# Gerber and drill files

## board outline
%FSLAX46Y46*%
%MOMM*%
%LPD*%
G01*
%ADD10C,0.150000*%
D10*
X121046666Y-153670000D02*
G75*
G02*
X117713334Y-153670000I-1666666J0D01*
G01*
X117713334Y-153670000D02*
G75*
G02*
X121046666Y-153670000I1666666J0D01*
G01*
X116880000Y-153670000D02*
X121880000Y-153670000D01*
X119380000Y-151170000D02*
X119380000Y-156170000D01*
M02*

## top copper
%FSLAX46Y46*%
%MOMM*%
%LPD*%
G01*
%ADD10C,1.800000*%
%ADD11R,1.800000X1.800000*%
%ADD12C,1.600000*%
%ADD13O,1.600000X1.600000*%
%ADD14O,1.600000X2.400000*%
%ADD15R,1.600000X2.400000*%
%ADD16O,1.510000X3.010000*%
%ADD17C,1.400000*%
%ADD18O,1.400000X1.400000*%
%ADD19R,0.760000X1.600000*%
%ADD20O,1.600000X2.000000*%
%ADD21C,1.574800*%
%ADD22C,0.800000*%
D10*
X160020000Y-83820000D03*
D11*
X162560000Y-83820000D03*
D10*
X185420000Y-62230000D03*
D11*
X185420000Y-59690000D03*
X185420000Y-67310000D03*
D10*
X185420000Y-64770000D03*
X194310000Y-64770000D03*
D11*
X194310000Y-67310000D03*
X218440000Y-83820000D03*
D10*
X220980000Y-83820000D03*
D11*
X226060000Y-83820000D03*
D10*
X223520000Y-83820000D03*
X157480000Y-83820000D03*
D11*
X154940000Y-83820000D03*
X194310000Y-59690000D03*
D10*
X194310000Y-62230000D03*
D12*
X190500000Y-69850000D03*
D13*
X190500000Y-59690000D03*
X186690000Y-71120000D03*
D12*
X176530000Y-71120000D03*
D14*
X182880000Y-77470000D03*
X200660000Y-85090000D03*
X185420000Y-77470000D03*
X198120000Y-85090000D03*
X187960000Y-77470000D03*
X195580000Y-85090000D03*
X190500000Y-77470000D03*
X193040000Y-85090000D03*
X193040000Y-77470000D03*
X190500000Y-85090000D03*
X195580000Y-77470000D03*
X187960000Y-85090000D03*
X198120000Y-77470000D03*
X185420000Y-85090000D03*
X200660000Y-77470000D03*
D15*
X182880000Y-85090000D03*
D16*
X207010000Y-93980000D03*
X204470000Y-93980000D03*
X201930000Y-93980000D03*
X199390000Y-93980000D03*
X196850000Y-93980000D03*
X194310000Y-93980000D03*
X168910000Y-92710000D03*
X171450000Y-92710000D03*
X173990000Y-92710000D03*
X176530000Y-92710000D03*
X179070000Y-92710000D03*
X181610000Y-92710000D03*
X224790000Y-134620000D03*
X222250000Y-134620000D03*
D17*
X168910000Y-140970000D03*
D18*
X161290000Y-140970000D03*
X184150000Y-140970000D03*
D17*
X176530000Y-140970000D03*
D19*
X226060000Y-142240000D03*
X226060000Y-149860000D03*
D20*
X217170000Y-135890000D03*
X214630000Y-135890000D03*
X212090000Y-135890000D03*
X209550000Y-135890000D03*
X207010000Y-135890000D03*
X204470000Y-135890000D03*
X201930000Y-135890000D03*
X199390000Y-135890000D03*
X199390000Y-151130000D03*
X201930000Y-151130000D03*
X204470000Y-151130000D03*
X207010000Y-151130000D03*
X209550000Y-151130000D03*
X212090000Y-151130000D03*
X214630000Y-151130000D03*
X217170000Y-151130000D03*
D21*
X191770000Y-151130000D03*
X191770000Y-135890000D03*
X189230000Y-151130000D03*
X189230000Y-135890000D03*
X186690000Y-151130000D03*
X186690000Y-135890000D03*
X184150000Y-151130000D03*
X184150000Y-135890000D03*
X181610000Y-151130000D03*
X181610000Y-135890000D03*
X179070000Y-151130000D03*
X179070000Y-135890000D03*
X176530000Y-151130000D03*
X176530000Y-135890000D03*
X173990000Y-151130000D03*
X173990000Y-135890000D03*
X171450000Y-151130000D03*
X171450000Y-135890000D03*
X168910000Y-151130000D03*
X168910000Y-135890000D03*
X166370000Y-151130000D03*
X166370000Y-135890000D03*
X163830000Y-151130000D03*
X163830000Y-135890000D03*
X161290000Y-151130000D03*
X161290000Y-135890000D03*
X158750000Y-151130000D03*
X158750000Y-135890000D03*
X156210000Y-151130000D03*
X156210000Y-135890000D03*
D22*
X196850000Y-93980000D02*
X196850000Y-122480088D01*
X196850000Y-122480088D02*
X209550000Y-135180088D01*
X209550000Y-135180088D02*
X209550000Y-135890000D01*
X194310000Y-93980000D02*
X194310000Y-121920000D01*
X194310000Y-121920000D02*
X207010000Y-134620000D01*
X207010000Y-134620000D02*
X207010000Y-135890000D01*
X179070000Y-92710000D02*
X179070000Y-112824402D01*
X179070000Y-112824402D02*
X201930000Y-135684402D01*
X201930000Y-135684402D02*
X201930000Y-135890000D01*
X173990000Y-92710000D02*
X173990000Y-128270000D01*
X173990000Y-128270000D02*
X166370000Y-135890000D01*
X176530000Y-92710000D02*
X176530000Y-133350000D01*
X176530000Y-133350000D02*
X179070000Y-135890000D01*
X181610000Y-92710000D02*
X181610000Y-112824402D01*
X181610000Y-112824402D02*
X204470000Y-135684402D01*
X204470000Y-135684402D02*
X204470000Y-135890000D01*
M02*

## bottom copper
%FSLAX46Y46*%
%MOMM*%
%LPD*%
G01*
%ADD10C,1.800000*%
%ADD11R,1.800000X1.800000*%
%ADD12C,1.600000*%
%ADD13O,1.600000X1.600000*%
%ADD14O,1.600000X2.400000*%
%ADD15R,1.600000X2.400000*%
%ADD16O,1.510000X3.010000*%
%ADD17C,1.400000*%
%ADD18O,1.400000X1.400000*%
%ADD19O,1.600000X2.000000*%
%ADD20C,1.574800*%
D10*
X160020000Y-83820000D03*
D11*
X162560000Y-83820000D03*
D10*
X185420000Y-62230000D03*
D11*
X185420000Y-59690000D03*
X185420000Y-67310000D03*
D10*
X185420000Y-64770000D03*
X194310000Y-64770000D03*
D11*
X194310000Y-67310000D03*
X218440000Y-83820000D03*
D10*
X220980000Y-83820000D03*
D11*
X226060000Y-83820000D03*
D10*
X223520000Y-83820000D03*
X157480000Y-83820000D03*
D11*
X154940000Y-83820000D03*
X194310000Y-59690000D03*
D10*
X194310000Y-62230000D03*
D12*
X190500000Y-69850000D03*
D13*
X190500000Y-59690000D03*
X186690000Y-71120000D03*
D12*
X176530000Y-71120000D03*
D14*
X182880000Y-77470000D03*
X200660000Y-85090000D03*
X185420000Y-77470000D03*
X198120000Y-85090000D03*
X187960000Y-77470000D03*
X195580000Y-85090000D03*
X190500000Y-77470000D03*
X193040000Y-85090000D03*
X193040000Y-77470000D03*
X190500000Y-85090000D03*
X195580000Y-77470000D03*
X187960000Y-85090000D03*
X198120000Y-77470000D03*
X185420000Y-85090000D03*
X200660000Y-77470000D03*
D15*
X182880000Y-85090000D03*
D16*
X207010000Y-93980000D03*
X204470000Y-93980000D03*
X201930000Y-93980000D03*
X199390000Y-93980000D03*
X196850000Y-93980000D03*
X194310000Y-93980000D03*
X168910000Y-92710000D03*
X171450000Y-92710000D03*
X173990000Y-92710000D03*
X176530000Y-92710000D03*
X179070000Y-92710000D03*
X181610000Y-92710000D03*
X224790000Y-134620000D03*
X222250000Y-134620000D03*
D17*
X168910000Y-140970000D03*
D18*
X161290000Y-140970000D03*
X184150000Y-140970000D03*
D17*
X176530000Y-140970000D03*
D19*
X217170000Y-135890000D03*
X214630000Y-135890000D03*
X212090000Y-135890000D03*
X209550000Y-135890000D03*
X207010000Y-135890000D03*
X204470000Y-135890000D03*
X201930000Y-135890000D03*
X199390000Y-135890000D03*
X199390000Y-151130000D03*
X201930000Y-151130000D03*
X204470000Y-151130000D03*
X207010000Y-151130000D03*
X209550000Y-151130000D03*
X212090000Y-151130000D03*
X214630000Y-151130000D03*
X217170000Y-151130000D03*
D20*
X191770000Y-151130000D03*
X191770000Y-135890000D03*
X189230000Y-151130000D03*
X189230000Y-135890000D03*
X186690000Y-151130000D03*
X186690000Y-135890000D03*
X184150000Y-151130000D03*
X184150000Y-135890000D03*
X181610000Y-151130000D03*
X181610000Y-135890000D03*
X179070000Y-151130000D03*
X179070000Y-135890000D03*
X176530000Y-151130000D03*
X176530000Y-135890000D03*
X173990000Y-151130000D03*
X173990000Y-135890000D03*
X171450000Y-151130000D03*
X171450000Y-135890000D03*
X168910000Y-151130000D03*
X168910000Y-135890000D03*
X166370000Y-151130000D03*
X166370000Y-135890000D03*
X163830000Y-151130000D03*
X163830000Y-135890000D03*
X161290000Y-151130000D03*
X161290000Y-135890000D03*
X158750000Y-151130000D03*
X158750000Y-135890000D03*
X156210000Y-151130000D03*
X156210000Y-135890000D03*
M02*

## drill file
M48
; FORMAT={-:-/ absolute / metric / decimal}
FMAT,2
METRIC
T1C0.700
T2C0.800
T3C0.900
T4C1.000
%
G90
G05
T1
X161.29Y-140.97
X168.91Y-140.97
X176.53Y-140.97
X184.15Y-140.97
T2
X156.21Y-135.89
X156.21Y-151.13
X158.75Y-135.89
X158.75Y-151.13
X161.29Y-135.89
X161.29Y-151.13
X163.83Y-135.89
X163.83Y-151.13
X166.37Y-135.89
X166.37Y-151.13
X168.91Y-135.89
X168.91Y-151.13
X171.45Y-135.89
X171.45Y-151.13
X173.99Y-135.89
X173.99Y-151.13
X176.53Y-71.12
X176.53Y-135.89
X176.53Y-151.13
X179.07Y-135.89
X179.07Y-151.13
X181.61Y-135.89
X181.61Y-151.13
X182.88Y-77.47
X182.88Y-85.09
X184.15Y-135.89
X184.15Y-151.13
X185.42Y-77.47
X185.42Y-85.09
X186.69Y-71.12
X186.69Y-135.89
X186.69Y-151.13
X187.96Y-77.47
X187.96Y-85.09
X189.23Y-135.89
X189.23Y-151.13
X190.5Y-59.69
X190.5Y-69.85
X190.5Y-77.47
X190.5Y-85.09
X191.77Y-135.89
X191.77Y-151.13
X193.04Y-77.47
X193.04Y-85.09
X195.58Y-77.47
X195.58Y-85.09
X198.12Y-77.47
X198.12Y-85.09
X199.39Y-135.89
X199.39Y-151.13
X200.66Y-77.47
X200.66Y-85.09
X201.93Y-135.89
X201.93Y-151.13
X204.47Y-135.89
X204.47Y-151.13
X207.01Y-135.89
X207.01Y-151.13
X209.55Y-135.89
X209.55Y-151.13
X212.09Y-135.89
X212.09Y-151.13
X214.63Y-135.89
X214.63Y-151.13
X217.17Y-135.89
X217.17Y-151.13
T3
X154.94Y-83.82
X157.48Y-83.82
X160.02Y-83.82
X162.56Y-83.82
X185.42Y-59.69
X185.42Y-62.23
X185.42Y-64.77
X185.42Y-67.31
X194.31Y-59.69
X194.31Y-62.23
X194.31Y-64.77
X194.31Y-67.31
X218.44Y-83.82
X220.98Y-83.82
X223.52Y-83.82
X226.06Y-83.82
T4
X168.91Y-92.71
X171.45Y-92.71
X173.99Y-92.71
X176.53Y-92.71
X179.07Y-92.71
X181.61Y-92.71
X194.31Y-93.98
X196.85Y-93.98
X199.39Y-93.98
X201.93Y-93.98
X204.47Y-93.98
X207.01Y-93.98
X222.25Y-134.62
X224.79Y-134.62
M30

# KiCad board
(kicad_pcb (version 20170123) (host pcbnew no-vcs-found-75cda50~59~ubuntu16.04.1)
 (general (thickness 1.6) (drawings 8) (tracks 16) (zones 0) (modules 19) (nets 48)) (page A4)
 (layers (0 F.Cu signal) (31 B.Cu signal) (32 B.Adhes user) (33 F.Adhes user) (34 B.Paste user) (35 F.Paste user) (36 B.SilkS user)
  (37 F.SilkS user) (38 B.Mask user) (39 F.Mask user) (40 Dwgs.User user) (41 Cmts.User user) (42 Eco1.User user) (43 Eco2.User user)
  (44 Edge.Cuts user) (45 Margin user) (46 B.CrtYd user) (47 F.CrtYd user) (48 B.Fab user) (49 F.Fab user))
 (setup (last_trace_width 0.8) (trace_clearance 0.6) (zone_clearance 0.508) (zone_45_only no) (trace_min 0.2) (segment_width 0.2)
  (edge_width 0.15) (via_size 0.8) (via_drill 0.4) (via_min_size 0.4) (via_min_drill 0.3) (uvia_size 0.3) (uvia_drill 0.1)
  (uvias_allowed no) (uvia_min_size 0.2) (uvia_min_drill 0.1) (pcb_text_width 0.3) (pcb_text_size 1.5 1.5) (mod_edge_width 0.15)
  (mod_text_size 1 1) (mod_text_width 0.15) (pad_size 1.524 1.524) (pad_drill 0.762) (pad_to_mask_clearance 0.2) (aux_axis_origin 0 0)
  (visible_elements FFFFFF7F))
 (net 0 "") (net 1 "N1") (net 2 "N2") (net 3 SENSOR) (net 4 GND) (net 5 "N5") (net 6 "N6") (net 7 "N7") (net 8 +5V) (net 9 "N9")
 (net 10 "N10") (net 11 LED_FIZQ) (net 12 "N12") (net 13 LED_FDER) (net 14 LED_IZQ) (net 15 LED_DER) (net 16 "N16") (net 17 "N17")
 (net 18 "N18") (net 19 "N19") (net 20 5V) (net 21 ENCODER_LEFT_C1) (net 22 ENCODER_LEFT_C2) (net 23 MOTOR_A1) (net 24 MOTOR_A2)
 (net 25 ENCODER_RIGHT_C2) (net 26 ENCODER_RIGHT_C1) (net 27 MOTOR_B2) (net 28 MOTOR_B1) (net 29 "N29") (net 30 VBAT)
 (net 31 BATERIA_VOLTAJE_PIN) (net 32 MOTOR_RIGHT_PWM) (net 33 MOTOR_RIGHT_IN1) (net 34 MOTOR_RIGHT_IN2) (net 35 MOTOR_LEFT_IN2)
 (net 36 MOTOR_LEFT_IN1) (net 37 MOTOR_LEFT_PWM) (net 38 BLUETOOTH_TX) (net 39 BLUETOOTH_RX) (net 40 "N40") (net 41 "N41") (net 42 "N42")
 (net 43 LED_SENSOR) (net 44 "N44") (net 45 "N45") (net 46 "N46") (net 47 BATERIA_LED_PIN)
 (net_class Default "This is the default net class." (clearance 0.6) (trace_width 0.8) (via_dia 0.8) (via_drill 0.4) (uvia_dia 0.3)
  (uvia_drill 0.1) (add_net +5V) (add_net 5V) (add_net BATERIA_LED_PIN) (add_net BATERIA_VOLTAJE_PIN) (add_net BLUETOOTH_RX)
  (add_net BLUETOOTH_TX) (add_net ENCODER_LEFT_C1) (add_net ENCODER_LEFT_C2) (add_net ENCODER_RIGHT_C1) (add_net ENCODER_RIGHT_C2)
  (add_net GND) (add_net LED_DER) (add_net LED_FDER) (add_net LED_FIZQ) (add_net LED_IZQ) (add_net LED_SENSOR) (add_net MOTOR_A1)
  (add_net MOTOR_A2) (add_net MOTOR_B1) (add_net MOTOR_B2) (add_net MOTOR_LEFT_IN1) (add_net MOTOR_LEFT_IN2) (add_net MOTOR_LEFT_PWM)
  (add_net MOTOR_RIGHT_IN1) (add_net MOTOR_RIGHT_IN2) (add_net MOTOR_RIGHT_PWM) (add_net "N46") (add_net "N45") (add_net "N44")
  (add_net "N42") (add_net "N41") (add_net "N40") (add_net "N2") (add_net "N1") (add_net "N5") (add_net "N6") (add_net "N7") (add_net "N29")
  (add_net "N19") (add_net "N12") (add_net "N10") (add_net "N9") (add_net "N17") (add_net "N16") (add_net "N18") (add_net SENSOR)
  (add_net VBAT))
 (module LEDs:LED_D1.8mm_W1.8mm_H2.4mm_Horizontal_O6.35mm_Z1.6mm (layer F.Cu) (at 162.56 83.82 180)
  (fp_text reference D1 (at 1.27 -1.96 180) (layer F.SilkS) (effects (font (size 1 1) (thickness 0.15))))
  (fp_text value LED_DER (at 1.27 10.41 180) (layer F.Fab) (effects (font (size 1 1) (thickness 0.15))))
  (pad 2 thru_hole circle (at 2.54 0 180) (size 1.8 1.8) (drill 0.9) (layers *.Cu *.Mask) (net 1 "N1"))
  (pad 1 thru_hole rect (at 0 0 180) (size 1.8 1.8) (drill 0.9) (layers *.Cu *.Mask) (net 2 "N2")))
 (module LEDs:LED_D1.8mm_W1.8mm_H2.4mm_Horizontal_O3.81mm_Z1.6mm (layer F.Cu) (at 185.42 59.69 270)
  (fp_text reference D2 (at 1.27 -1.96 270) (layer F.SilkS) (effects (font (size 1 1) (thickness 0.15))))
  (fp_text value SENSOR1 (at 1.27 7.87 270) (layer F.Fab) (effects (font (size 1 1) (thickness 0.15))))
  (pad 2 thru_hole circle (at 2.54 0 270) (size 1.8 1.8) (drill 0.9) (layers *.Cu *.Mask) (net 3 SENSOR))
  (pad 1 thru_hole rect (at 0 0 270) (size 1.8 1.8) (drill 0.9) (layers *.Cu *.Mask) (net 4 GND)))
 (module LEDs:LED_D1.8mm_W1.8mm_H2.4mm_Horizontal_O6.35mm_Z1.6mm (layer B.Cu) (at 185.42 67.31 90)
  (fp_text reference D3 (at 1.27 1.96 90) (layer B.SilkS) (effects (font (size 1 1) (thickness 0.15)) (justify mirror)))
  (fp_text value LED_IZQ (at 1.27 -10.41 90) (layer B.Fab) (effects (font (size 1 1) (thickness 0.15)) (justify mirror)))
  (pad 1 thru_hole rect (at 0 0 90) (size 1.8 1.8) (drill 0.9) (layers *.Cu *.Mask) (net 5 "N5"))
  (pad 2 thru_hole circle (at 2.54 0 90) (size 1.8 1.8) (drill 0.9) (layers *.Cu *.Mask) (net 1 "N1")))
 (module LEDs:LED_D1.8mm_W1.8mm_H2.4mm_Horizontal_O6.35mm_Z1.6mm (layer F.Cu) (at 194.31 67.31 90)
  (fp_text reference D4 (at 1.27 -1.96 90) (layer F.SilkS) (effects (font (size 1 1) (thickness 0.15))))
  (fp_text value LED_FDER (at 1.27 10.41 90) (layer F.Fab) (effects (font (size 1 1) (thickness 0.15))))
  (pad 2 thru_hole circle (at 2.54 0 90) (size 1.8 1.8) (drill 0.9) (layers *.Cu *.Mask) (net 1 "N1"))
  (pad 1 thru_hole rect (at 0 0 90) (size 1.8 1.8) (drill 0.9) (layers *.Cu *.Mask) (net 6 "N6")))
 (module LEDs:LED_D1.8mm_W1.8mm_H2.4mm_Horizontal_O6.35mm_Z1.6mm (layer B.Cu) (at 218.44 83.82)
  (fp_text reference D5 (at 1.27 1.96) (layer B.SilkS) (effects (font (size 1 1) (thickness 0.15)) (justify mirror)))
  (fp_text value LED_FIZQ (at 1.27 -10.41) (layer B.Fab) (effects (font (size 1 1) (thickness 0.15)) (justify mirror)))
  (pad 1 thru_hole rect (at 0 0) (size 1.8 1.8) (drill 0.9) (layers *.Cu *.Mask) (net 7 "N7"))
  (pad 2 thru_hole circle (at 2.54 0) (size 1.8 1.8) (drill 0.9) (layers *.Cu *.Mask) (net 1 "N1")))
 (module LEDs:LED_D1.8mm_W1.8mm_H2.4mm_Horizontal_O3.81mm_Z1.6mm (layer F.Cu) (at 226.06 83.82 180)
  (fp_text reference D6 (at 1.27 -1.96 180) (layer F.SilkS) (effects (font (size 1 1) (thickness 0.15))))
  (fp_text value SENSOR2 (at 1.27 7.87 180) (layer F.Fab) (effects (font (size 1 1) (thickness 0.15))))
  (pad 1 thru_hole rect (at 0 0 180) (size 1.8 1.8) (drill 0.9) (layers *.Cu *.Mask) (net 4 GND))
  (pad 2 thru_hole circle (at 2.54 0 180) (size 1.8 1.8) (drill 0.9) (layers *.Cu *.Mask) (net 3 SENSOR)))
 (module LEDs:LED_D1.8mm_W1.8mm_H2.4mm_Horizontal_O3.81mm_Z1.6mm (layer B.Cu) (at 154.94 83.82)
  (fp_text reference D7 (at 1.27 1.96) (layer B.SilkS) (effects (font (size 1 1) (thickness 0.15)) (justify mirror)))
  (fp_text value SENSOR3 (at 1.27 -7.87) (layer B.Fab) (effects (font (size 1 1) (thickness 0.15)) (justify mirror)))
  (pad 2 thru_hole circle (at 2.54 0) (size 1.8 1.8) (drill 0.9) (layers *.Cu *.Mask) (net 3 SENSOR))
  (pad 1 thru_hole rect (at 0 0) (size 1.8 1.8) (drill 0.9) (layers *.Cu *.Mask) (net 4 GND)))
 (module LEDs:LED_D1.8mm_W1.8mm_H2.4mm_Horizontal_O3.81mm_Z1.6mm (layer B.Cu) (at 194.31 59.69 270)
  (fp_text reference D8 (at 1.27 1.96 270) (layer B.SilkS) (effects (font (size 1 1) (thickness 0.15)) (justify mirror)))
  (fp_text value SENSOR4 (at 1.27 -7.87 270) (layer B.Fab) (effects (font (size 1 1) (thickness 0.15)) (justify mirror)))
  (pad 1 thru_hole rect (at 0 0 270) (size 1.8 1.8) (drill 0.9) (layers *.Cu *.Mask) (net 4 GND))
  (pad 2 thru_hole circle (at 2.54 0 270) (size 1.8 1.8) (drill 0.9) (layers *.Cu *.Mask) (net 3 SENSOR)))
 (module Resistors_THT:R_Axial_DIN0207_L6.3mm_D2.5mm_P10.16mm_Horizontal (layer F.Cu) (at 190.5 69.85 90)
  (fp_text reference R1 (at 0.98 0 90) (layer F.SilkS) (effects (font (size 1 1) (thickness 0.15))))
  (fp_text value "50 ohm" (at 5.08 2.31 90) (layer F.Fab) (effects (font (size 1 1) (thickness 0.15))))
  (pad 1 thru_hole circle (at 0 0 90) (size 1.6 1.6) (drill 0.8) (layers *.Cu *.Mask) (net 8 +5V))
  (pad 2 thru_hole oval (at 10.16 0 90) (size 1.6 1.6) (drill 0.8) (layers *.Cu *.Mask) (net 1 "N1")))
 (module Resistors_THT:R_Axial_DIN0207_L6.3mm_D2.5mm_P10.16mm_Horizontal (layer F.Cu) (at 176.53 71.12)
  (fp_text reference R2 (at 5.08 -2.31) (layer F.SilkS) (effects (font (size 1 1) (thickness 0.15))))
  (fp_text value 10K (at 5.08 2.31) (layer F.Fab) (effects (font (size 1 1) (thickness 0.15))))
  (pad 2 thru_hole oval (at 10.16 0) (size 1.6 1.6) (drill 0.8) (layers *.Cu *.Mask) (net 8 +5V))
  (pad 1 thru_hole circle (at 0 0) (size 1.6 1.6) (drill 0.8) (layers *.Cu *.Mask) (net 3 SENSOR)))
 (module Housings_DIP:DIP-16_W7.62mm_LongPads (layer F.Cu) (at 182.88 85.09 90)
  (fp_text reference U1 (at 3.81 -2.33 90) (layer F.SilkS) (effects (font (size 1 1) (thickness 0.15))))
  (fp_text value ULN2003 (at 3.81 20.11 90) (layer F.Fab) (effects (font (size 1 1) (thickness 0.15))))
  (pad 16 thru_hole oval (at 7.62 0 90) (size 2.4 1.6) (drill 0.8) (layers *.Cu *.Mask) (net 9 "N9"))
  (pad 8 thru_hole oval (at 0 17.78 90) (size 2.4 1.6) (drill 0.8) (layers *.Cu *.Mask) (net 4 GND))
  (pad 15 thru_hole oval (at 7.62 2.54 90) (size 2.4 1.6) (drill 0.8) (layers *.Cu *.Mask) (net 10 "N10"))
  (pad 7 thru_hole oval (at 0 15.24 90) (size 2.4 1.6) (drill 0.8) (layers *.Cu *.Mask) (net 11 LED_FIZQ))
  (pad 14 thru_hole oval (at 7.62 5.08 90) (size 2.4 1.6) (drill 0.8) (layers *.Cu *.Mask) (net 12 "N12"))
  (pad 6 thru_hole oval (at 0 12.7 90) (size 2.4 1.6) (drill 0.8) (layers *.Cu *.Mask) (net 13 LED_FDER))
  (pad 13 thru_hole oval (at 7.62 7.62 90) (size 2.4 1.6) (drill 0.8) (layers *.Cu *.Mask) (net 2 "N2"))
  (pad 5 thru_hole oval (at 0 10.16 90) (size 2.4 1.6) (drill 0.8) (layers *.Cu *.Mask) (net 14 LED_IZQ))
  (pad 12 thru_hole oval (at 7.62 10.16 90) (size 2.4 1.6) (drill 0.8) (layers *.Cu *.Mask) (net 5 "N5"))
  (pad 4 thru_hole oval (at 0 7.62 90) (size 2.4 1.6) (drill 0.8) (layers *.Cu *.Mask) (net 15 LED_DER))
  (pad 11 thru_hole oval (at 7.62 12.7 90) (size 2.4 1.6) (drill 0.8) (layers *.Cu *.Mask) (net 6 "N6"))
  (pad 3 thru_hole oval (at 0 5.08 90) (size 2.4 1.6) (drill 0.8) (layers *.Cu *.Mask) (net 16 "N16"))
  (pad 10 thru_hole oval (at 7.62 15.24 90) (size 2.4 1.6) (drill 0.8) (layers *.Cu *.Mask) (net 7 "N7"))
  (pad 2 thru_hole oval (at 0 2.54 90) (size 2.4 1.6) (drill 0.8) (layers *.Cu *.Mask) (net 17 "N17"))
  (pad 9 thru_hole oval (at 7.62 17.78 90) (size 2.4 1.6) (drill 0.8) (layers *.Cu *.Mask) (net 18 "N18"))
  (pad 1 thru_hole rect (at 0 0 90) (size 2.4 1.6) (drill 0.8) (layers *.Cu *.Mask) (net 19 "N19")))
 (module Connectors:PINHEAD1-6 (layer F.Cu) (at 194.31 93.98)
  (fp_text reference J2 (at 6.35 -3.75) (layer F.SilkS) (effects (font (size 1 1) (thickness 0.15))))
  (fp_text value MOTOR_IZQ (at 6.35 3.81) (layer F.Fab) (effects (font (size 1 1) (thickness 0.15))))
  (pad 6 thru_hole oval (at 12.7 0) (size 1.51 3.01) (drill 1) (layers *.Cu *.Mask) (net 4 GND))
  (pad 5 thru_hole oval (at 10.16 0) (size 1.51 3.01) (drill 1) (layers *.Cu *.Mask) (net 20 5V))
  (pad 4 thru_hole oval (at 7.62 0) (size 1.51 3.01) (drill 1) (layers *.Cu *.Mask) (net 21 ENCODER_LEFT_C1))
  (pad 3 thru_hole oval (at 5.08 0) (size 1.51 3.01) (drill 1) (layers *.Cu *.Mask) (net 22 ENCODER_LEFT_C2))
  (pad 2 thru_hole oval (at 2.54 0) (size 1.51 3.01) (drill 1) (layers *.Cu *.Mask) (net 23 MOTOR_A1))
  (pad 1 thru_hole oval (at 0 0) (size 1.51 3.01) (drill 1) (layers *.Cu *.Mask) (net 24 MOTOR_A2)))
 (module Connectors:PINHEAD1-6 (layer F.Cu) (at 168.91 92.71)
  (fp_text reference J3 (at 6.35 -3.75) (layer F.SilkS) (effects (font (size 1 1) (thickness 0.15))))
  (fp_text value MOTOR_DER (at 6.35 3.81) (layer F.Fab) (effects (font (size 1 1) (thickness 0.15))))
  (pad 1 thru_hole oval (at 0 0) (size 1.51 3.01) (drill 1) (layers *.Cu *.Mask) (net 4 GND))
  (pad 2 thru_hole oval (at 2.54 0) (size 1.51 3.01) (drill 1) (layers *.Cu *.Mask) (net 20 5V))
  (pad 3 thru_hole oval (at 5.08 0) (size 1.51 3.01) (drill 1) (layers *.Cu *.Mask) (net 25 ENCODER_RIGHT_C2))
  (pad 4 thru_hole oval (at 7.62 0) (size 1.51 3.01) (drill 1) (layers *.Cu *.Mask) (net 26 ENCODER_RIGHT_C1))
  (pad 5 thru_hole oval (at 10.16 0) (size 1.51 3.01) (drill 1) (layers *.Cu *.Mask) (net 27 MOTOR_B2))
  (pad 6 thru_hole oval (at 12.7 0) (size 1.51 3.01) (drill 1) (layers *.Cu *.Mask) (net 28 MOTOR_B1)))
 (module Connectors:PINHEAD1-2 (layer F.Cu) (at 222.25 134.62)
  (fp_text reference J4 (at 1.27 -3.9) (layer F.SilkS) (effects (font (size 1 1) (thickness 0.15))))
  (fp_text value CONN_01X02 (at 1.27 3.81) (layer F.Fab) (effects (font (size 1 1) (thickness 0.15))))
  (pad 2 thru_hole oval (at 2.54 0) (size 1.51 3.01) (drill 1) (layers *.Cu *.Mask) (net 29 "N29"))
  (pad 1 thru_hole oval (at 0 0) (size 1.51 3.01) (drill 1) (layers *.Cu *.Mask) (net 4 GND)))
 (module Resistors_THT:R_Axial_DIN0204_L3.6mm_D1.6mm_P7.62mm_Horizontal (layer F.Cu) (at 168.91 140.97 180)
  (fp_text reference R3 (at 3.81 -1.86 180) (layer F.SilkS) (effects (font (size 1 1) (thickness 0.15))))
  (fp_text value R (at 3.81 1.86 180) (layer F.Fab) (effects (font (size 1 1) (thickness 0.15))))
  (pad 1 thru_hole circle (at 0 0 180) (size 1.4 1.4) (drill 0.7) (layers *.Cu *.Mask) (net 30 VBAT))
  (pad 2 thru_hole oval (at 7.62 0 180) (size 1.4 1.4) (drill 0.7) (layers *.Cu *.Mask) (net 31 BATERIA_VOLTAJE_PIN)))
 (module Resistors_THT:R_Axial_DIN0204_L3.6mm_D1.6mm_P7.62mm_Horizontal (layer F.Cu) (at 176.53 140.97)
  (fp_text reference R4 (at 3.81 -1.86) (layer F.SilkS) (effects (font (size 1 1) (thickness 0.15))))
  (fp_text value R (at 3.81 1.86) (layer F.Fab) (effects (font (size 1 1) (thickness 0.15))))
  (pad 2 thru_hole oval (at 7.62 0) (size 1.4 1.4) (drill 0.7) (layers *.Cu *.Mask) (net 4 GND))
  (pad 1 thru_hole circle (at 0 0) (size 1.4 1.4) (drill 0.7) (layers *.Cu *.Mask) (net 31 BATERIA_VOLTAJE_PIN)))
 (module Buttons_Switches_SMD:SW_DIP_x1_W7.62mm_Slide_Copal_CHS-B (layer F.Cu) (at 226.06 146.05 90)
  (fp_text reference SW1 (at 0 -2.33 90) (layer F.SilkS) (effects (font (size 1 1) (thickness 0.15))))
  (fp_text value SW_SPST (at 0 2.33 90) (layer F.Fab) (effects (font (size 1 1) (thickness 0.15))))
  (pad 2 smd rect (at 3.81 0 90) (size 1.6 0.76) (layers F.Cu F.Paste F.Mask) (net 30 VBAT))
  (pad 1 smd rect (at -3.81 0 90) (size 1.6 0.76) (layers F.Cu F.Paste F.Mask) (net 29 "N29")))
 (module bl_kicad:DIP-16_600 (layer F.Cu) (at 217.17 135.89 270)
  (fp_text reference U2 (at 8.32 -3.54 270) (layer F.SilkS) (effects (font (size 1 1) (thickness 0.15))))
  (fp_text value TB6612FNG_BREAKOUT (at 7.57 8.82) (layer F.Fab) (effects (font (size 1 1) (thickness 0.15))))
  (pad 1 thru_hole oval (at 0 0 270) (size 2 1.6) (drill 0.8) (layers *.Cu *.Mask F.SilkS) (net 30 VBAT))
  (pad 2 thru_hole oval (at 0 2.54 270) (size 2 1.6) (drill 0.8) (layers *.Cu *.Mask F.SilkS) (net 20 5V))
  (pad 3 thru_hole oval (at 0 5.08 270) (size 2 1.6) (drill 0.8) (layers *.Cu *.Mask F.SilkS) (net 4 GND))
  (pad 4 thru_hole oval (at 0 7.62 270) (size 2 1.6) (drill 0.8) (layers *.Cu *.Mask F.SilkS) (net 23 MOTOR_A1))
  (pad 5 thru_hole oval (at 0 10.16 270) (size 2 1.6) (drill 0.8) (layers *.Cu *.Mask F.SilkS) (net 24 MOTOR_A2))
  (pad 6 thru_hole oval (at 0 12.7 270) (size 2 1.6) (drill 0.8) (layers *.Cu *.Mask F.SilkS) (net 28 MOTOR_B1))
  (pad 7 thru_hole oval (at 0 15.24 270) (size 2 1.6) (drill 0.8) (layers *.Cu *.Mask F.SilkS) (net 27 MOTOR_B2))
  (pad 8 thru_hole oval (at 0 17.78 270) (size 2 1.6) (drill 0.8) (layers *.Cu *.Mask F.SilkS) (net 4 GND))
  (pad 9 thru_hole oval (at 15.24 17.78 270) (size 2 1.6) (drill 0.8) (layers *.Cu *.Mask F.SilkS) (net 4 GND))
  (pad 10 thru_hole oval (at 15.24 15.24 270) (size 2 1.6) (drill 0.8) (layers *.Cu *.Mask F.SilkS) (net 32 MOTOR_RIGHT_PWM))
  (pad 11 thru_hole oval (at 15.24 12.7 270) (size 2 1.6) (drill 0.8) (layers *.Cu *.Mask F.SilkS) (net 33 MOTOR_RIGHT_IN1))
  (pad 12 thru_hole oval (at 15.24 10.16 270) (size 2 1.6) (drill 0.8) (layers *.Cu *.Mask F.SilkS) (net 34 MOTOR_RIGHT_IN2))
  (pad 13 thru_hole oval (at 15.24 7.62 270) (size 2 1.6) (drill 0.8) (layers *.Cu *.Mask F.SilkS) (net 20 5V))
  (pad 14 thru_hole oval (at 15.24 5.08 270) (size 2 1.6) (drill 0.8) (layers *.Cu *.Mask F.SilkS) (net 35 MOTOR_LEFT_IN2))
  (pad 15 thru_hole oval (at 15.24 2.54 270) (size 2 1.6) (drill 0.8) (layers *.Cu *.Mask F.SilkS) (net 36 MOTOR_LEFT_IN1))
  (pad 16 thru_hole oval (at 15.24 0 270) (size 2 1.6) (drill 0.8) (layers *.Cu *.Mask F.SilkS) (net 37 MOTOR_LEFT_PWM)))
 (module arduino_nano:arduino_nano (layer F.Cu) (at 173.99 143.51 180)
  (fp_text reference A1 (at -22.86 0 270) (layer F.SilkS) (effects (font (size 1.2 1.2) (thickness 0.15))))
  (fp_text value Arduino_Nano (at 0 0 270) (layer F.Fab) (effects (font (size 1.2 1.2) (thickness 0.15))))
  (pad 30 thru_hole circle (at -17.78 -7.62 180) (size 1.5748 1.5748) (drill 0.8) (layers *.Cu *.Mask F.SilkS) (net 30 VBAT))
  (pad 1 thru_hole circle (at -17.78 7.62 180) (size 1.5748 1.5748) (drill 0.8) (layers *.Cu *.Mask F.SilkS) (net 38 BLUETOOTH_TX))
  (pad 29 thru_hole circle (at -15.24 -7.62 180) (size 1.5748 1.5748) (drill 0.8) (layers *.Cu *.Mask F.SilkS) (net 4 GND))
  (pad 2 thru_hole circle (at -15.24 7.62 180) (size 1.5748 1.5748) (drill 0.8) (layers *.Cu *.Mask F.SilkS) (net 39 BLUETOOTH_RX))
  (pad 28 thru_hole circle (at -12.7 -7.62 180) (size 1.5748 1.5748) (drill 0.8) (layers *.Cu *.Mask F.SilkS))
  (pad 3 thru_hole circle (at -12.7 7.62 180) (size 1.5748 1.5748) (drill 0.8) (layers *.Cu *.Mask F.SilkS) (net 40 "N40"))
  (pad 27 thru_hole circle (at -10.16 -7.62 180) (size 1.5748 1.5748) (drill 0.8) (layers *.Cu *.Mask F.SilkS) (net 20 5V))
  (pad 4 thru_hole circle (at -10.16 7.62 180) (size 1.5748 1.5748) (drill 0.8) (layers *.Cu *.Mask F.SilkS) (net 4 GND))
  (pad 26 thru_hole circle (at -7.62 -7.62 180) (size 1.5748 1.5748) (drill 0.8) (layers *.Cu *.Mask F.SilkS) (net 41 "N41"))
  (pad 5 thru_hole circle (at -7.62 7.62 180) (size 1.5748 1.5748) (drill 0.8) (layers *.Cu *.Mask F.SilkS) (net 21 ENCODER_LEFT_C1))
  (pad 25 thru_hole circle (at -5.08 -7.62 180) (size 1.5748 1.5748) (drill 0.8) (layers *.Cu *.Mask F.SilkS) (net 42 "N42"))
  (pad 6 thru_hole circle (at -5.08 7.62 180) (size 1.5748 1.5748) (drill 0.8) (layers *.Cu *.Mask F.SilkS) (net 26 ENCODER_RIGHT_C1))
  (pad 24 thru_hole circle (at -2.54 -7.62 180) (size 1.5748 1.5748) (drill 0.8) (layers *.Cu *.Mask F.SilkS) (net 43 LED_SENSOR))
  (pad 7 thru_hole circle (at -2.54 7.62 180) (size 1.5748 1.5748) (drill 0.8) (layers *.Cu *.Mask F.SilkS) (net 35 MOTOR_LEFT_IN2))
  (pad 23 thru_hole circle (at 0 -7.62 180) (size 1.5748 1.5748) (drill 0.8) (layers *.Cu *.Mask F.SilkS) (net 13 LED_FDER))
  (pad 8 thru_hole circle (at 0 7.62 180) (size 1.5748 1.5748) (drill 0.8) (layers *.Cu *.Mask F.SilkS) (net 37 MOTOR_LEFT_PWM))
  (pad 22 thru_hole circle (at 2.54 -7.62 180) (size 1.5748 1.5748) (drill 0.8) (layers *.Cu *.Mask F.SilkS) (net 11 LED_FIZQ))
  (pad 9 thru_hole circle (at 2.54 7.62 180) (size 1.5748 1.5748) (drill 0.8) (layers *.Cu *.Mask F.SilkS) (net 32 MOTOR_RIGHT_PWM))
  (pad 21 thru_hole circle (at 5.08 -7.62 180) (size 1.5748 1.5748) (drill 0.8) (layers *.Cu *.Mask F.SilkS) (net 15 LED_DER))
  (pad 10 thru_hole circle (at 5.08 7.62 180) (size 1.5748 1.5748) (drill 0.8) (layers *.Cu *.Mask F.SilkS) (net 33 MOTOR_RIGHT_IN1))
  (pad 20 thru_hole circle (at 7.62 -7.62 180) (size 1.5748 1.5748) (drill 0.8) (layers *.Cu *.Mask F.SilkS) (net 14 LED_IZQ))
  (pad 11 thru_hole circle (at 7.62 7.62 180) (size 1.5748 1.5748) (drill 0.8) (layers *.Cu *.Mask F.SilkS) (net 25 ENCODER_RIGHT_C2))
  (pad 19 thru_hole circle (at 10.16 -7.62 180) (size 1.5748 1.5748) (drill 0.8) (layers *.Cu *.Mask F.SilkS) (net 31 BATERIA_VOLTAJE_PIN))
  (pad 12 thru_hole circle (at 10.16 7.62 180) (size 1.5748 1.5748) (drill 0.8) (layers *.Cu *.Mask F.SilkS) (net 36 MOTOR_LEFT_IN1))
  (pad 18 thru_hole circle (at 12.7 -7.62 180) (size 1.5748 1.5748) (drill 0.8) (layers *.Cu *.Mask F.SilkS) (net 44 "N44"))
  (pad 13 thru_hole circle (at 12.7 7.62 180) (size 1.5748 1.5748) (drill 0.8) (layers *.Cu *.Mask F.SilkS) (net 34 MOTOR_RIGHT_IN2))
  (pad 17 thru_hole circle (at 15.24 -7.62 180) (size 1.5748 1.5748) (drill 0.8) (layers *.Cu *.Mask F.SilkS) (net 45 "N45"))
  (pad 14 thru_hole circle (at 15.24 7.62 180) (size 1.5748 1.5748) (drill 0.8) (layers *.Cu *.Mask F.SilkS) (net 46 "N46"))
  (pad 16 thru_hole circle (at 17.78 -7.62 180) (size 1.5748 1.5748) (drill 0.8) (layers *.Cu *.Mask F.SilkS) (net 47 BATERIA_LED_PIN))
  (pad 15 thru_hole circle (at 17.78 7.62 180) (size 1.5748 1.5748) (drill 0.8) (layers *.Cu *.Mask F.SilkS) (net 22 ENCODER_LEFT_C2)))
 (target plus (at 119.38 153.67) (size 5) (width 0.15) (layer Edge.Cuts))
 (segment (start 196.85 93.98) (end 196.85 122.480088) (width 0.8) (layer F.Cu) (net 23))
 (segment (start 196.85 122.480088) (end 209.55 135.180088) (width 0.8) (layer F.Cu) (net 23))
 (segment (start 209.55 135.180088) (end 209.55 135.89) (width 0.8) (layer F.Cu) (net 23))
 (segment (start 194.31 93.98) (end 194.31 121.92) (width 0.8) (layer F.Cu) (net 24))
 (segment (start 194.31 121.92) (end 207.01 134.62) (width 0.8) (layer F.Cu) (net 24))
 (segment (start 207.01 134.62) (end 207.01 135.89) (width 0.8) (layer F.Cu) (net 24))
 (segment (start 179.07 92.71) (end 179.07 112.824402) (width 0.8) (layer F.Cu) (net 27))
 (segment (start 179.07 112.824402) (end 201.93 135.684402) (width 0.8) (layer F.Cu) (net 27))
 (segment (start 201.93 135.684402) (end 201.93 135.89) (width 0.8) (layer F.Cu) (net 27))
 (segment (start 173.99 92.71) (end 173.99 128.27) (width 0.8) (layer F.Cu) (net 25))
 (segment (start 173.99 128.27) (end 166.37 135.89) (width 0.8) (layer F.Cu) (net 25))
 (segment (start 176.53 92.71) (end 176.53 133.35) (width 0.8) (layer F.Cu) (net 26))
 (segment (start 176.53 133.35) (end 179.07 135.89) (width 0.8) (layer F.Cu) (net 26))
 (segment (start 181.61 92.71) (end 181.61 112.824402) (width 0.8) (layer F.Cu) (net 28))
 (segment (start 181.61 112.824402) (end 204.47 135.684402) (width 0.8) (layer F.Cu) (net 28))
 (segment (start 204.47 135.684402) (end 204.47 135.89) (width 0.8) (layer F.Cu) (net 28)))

